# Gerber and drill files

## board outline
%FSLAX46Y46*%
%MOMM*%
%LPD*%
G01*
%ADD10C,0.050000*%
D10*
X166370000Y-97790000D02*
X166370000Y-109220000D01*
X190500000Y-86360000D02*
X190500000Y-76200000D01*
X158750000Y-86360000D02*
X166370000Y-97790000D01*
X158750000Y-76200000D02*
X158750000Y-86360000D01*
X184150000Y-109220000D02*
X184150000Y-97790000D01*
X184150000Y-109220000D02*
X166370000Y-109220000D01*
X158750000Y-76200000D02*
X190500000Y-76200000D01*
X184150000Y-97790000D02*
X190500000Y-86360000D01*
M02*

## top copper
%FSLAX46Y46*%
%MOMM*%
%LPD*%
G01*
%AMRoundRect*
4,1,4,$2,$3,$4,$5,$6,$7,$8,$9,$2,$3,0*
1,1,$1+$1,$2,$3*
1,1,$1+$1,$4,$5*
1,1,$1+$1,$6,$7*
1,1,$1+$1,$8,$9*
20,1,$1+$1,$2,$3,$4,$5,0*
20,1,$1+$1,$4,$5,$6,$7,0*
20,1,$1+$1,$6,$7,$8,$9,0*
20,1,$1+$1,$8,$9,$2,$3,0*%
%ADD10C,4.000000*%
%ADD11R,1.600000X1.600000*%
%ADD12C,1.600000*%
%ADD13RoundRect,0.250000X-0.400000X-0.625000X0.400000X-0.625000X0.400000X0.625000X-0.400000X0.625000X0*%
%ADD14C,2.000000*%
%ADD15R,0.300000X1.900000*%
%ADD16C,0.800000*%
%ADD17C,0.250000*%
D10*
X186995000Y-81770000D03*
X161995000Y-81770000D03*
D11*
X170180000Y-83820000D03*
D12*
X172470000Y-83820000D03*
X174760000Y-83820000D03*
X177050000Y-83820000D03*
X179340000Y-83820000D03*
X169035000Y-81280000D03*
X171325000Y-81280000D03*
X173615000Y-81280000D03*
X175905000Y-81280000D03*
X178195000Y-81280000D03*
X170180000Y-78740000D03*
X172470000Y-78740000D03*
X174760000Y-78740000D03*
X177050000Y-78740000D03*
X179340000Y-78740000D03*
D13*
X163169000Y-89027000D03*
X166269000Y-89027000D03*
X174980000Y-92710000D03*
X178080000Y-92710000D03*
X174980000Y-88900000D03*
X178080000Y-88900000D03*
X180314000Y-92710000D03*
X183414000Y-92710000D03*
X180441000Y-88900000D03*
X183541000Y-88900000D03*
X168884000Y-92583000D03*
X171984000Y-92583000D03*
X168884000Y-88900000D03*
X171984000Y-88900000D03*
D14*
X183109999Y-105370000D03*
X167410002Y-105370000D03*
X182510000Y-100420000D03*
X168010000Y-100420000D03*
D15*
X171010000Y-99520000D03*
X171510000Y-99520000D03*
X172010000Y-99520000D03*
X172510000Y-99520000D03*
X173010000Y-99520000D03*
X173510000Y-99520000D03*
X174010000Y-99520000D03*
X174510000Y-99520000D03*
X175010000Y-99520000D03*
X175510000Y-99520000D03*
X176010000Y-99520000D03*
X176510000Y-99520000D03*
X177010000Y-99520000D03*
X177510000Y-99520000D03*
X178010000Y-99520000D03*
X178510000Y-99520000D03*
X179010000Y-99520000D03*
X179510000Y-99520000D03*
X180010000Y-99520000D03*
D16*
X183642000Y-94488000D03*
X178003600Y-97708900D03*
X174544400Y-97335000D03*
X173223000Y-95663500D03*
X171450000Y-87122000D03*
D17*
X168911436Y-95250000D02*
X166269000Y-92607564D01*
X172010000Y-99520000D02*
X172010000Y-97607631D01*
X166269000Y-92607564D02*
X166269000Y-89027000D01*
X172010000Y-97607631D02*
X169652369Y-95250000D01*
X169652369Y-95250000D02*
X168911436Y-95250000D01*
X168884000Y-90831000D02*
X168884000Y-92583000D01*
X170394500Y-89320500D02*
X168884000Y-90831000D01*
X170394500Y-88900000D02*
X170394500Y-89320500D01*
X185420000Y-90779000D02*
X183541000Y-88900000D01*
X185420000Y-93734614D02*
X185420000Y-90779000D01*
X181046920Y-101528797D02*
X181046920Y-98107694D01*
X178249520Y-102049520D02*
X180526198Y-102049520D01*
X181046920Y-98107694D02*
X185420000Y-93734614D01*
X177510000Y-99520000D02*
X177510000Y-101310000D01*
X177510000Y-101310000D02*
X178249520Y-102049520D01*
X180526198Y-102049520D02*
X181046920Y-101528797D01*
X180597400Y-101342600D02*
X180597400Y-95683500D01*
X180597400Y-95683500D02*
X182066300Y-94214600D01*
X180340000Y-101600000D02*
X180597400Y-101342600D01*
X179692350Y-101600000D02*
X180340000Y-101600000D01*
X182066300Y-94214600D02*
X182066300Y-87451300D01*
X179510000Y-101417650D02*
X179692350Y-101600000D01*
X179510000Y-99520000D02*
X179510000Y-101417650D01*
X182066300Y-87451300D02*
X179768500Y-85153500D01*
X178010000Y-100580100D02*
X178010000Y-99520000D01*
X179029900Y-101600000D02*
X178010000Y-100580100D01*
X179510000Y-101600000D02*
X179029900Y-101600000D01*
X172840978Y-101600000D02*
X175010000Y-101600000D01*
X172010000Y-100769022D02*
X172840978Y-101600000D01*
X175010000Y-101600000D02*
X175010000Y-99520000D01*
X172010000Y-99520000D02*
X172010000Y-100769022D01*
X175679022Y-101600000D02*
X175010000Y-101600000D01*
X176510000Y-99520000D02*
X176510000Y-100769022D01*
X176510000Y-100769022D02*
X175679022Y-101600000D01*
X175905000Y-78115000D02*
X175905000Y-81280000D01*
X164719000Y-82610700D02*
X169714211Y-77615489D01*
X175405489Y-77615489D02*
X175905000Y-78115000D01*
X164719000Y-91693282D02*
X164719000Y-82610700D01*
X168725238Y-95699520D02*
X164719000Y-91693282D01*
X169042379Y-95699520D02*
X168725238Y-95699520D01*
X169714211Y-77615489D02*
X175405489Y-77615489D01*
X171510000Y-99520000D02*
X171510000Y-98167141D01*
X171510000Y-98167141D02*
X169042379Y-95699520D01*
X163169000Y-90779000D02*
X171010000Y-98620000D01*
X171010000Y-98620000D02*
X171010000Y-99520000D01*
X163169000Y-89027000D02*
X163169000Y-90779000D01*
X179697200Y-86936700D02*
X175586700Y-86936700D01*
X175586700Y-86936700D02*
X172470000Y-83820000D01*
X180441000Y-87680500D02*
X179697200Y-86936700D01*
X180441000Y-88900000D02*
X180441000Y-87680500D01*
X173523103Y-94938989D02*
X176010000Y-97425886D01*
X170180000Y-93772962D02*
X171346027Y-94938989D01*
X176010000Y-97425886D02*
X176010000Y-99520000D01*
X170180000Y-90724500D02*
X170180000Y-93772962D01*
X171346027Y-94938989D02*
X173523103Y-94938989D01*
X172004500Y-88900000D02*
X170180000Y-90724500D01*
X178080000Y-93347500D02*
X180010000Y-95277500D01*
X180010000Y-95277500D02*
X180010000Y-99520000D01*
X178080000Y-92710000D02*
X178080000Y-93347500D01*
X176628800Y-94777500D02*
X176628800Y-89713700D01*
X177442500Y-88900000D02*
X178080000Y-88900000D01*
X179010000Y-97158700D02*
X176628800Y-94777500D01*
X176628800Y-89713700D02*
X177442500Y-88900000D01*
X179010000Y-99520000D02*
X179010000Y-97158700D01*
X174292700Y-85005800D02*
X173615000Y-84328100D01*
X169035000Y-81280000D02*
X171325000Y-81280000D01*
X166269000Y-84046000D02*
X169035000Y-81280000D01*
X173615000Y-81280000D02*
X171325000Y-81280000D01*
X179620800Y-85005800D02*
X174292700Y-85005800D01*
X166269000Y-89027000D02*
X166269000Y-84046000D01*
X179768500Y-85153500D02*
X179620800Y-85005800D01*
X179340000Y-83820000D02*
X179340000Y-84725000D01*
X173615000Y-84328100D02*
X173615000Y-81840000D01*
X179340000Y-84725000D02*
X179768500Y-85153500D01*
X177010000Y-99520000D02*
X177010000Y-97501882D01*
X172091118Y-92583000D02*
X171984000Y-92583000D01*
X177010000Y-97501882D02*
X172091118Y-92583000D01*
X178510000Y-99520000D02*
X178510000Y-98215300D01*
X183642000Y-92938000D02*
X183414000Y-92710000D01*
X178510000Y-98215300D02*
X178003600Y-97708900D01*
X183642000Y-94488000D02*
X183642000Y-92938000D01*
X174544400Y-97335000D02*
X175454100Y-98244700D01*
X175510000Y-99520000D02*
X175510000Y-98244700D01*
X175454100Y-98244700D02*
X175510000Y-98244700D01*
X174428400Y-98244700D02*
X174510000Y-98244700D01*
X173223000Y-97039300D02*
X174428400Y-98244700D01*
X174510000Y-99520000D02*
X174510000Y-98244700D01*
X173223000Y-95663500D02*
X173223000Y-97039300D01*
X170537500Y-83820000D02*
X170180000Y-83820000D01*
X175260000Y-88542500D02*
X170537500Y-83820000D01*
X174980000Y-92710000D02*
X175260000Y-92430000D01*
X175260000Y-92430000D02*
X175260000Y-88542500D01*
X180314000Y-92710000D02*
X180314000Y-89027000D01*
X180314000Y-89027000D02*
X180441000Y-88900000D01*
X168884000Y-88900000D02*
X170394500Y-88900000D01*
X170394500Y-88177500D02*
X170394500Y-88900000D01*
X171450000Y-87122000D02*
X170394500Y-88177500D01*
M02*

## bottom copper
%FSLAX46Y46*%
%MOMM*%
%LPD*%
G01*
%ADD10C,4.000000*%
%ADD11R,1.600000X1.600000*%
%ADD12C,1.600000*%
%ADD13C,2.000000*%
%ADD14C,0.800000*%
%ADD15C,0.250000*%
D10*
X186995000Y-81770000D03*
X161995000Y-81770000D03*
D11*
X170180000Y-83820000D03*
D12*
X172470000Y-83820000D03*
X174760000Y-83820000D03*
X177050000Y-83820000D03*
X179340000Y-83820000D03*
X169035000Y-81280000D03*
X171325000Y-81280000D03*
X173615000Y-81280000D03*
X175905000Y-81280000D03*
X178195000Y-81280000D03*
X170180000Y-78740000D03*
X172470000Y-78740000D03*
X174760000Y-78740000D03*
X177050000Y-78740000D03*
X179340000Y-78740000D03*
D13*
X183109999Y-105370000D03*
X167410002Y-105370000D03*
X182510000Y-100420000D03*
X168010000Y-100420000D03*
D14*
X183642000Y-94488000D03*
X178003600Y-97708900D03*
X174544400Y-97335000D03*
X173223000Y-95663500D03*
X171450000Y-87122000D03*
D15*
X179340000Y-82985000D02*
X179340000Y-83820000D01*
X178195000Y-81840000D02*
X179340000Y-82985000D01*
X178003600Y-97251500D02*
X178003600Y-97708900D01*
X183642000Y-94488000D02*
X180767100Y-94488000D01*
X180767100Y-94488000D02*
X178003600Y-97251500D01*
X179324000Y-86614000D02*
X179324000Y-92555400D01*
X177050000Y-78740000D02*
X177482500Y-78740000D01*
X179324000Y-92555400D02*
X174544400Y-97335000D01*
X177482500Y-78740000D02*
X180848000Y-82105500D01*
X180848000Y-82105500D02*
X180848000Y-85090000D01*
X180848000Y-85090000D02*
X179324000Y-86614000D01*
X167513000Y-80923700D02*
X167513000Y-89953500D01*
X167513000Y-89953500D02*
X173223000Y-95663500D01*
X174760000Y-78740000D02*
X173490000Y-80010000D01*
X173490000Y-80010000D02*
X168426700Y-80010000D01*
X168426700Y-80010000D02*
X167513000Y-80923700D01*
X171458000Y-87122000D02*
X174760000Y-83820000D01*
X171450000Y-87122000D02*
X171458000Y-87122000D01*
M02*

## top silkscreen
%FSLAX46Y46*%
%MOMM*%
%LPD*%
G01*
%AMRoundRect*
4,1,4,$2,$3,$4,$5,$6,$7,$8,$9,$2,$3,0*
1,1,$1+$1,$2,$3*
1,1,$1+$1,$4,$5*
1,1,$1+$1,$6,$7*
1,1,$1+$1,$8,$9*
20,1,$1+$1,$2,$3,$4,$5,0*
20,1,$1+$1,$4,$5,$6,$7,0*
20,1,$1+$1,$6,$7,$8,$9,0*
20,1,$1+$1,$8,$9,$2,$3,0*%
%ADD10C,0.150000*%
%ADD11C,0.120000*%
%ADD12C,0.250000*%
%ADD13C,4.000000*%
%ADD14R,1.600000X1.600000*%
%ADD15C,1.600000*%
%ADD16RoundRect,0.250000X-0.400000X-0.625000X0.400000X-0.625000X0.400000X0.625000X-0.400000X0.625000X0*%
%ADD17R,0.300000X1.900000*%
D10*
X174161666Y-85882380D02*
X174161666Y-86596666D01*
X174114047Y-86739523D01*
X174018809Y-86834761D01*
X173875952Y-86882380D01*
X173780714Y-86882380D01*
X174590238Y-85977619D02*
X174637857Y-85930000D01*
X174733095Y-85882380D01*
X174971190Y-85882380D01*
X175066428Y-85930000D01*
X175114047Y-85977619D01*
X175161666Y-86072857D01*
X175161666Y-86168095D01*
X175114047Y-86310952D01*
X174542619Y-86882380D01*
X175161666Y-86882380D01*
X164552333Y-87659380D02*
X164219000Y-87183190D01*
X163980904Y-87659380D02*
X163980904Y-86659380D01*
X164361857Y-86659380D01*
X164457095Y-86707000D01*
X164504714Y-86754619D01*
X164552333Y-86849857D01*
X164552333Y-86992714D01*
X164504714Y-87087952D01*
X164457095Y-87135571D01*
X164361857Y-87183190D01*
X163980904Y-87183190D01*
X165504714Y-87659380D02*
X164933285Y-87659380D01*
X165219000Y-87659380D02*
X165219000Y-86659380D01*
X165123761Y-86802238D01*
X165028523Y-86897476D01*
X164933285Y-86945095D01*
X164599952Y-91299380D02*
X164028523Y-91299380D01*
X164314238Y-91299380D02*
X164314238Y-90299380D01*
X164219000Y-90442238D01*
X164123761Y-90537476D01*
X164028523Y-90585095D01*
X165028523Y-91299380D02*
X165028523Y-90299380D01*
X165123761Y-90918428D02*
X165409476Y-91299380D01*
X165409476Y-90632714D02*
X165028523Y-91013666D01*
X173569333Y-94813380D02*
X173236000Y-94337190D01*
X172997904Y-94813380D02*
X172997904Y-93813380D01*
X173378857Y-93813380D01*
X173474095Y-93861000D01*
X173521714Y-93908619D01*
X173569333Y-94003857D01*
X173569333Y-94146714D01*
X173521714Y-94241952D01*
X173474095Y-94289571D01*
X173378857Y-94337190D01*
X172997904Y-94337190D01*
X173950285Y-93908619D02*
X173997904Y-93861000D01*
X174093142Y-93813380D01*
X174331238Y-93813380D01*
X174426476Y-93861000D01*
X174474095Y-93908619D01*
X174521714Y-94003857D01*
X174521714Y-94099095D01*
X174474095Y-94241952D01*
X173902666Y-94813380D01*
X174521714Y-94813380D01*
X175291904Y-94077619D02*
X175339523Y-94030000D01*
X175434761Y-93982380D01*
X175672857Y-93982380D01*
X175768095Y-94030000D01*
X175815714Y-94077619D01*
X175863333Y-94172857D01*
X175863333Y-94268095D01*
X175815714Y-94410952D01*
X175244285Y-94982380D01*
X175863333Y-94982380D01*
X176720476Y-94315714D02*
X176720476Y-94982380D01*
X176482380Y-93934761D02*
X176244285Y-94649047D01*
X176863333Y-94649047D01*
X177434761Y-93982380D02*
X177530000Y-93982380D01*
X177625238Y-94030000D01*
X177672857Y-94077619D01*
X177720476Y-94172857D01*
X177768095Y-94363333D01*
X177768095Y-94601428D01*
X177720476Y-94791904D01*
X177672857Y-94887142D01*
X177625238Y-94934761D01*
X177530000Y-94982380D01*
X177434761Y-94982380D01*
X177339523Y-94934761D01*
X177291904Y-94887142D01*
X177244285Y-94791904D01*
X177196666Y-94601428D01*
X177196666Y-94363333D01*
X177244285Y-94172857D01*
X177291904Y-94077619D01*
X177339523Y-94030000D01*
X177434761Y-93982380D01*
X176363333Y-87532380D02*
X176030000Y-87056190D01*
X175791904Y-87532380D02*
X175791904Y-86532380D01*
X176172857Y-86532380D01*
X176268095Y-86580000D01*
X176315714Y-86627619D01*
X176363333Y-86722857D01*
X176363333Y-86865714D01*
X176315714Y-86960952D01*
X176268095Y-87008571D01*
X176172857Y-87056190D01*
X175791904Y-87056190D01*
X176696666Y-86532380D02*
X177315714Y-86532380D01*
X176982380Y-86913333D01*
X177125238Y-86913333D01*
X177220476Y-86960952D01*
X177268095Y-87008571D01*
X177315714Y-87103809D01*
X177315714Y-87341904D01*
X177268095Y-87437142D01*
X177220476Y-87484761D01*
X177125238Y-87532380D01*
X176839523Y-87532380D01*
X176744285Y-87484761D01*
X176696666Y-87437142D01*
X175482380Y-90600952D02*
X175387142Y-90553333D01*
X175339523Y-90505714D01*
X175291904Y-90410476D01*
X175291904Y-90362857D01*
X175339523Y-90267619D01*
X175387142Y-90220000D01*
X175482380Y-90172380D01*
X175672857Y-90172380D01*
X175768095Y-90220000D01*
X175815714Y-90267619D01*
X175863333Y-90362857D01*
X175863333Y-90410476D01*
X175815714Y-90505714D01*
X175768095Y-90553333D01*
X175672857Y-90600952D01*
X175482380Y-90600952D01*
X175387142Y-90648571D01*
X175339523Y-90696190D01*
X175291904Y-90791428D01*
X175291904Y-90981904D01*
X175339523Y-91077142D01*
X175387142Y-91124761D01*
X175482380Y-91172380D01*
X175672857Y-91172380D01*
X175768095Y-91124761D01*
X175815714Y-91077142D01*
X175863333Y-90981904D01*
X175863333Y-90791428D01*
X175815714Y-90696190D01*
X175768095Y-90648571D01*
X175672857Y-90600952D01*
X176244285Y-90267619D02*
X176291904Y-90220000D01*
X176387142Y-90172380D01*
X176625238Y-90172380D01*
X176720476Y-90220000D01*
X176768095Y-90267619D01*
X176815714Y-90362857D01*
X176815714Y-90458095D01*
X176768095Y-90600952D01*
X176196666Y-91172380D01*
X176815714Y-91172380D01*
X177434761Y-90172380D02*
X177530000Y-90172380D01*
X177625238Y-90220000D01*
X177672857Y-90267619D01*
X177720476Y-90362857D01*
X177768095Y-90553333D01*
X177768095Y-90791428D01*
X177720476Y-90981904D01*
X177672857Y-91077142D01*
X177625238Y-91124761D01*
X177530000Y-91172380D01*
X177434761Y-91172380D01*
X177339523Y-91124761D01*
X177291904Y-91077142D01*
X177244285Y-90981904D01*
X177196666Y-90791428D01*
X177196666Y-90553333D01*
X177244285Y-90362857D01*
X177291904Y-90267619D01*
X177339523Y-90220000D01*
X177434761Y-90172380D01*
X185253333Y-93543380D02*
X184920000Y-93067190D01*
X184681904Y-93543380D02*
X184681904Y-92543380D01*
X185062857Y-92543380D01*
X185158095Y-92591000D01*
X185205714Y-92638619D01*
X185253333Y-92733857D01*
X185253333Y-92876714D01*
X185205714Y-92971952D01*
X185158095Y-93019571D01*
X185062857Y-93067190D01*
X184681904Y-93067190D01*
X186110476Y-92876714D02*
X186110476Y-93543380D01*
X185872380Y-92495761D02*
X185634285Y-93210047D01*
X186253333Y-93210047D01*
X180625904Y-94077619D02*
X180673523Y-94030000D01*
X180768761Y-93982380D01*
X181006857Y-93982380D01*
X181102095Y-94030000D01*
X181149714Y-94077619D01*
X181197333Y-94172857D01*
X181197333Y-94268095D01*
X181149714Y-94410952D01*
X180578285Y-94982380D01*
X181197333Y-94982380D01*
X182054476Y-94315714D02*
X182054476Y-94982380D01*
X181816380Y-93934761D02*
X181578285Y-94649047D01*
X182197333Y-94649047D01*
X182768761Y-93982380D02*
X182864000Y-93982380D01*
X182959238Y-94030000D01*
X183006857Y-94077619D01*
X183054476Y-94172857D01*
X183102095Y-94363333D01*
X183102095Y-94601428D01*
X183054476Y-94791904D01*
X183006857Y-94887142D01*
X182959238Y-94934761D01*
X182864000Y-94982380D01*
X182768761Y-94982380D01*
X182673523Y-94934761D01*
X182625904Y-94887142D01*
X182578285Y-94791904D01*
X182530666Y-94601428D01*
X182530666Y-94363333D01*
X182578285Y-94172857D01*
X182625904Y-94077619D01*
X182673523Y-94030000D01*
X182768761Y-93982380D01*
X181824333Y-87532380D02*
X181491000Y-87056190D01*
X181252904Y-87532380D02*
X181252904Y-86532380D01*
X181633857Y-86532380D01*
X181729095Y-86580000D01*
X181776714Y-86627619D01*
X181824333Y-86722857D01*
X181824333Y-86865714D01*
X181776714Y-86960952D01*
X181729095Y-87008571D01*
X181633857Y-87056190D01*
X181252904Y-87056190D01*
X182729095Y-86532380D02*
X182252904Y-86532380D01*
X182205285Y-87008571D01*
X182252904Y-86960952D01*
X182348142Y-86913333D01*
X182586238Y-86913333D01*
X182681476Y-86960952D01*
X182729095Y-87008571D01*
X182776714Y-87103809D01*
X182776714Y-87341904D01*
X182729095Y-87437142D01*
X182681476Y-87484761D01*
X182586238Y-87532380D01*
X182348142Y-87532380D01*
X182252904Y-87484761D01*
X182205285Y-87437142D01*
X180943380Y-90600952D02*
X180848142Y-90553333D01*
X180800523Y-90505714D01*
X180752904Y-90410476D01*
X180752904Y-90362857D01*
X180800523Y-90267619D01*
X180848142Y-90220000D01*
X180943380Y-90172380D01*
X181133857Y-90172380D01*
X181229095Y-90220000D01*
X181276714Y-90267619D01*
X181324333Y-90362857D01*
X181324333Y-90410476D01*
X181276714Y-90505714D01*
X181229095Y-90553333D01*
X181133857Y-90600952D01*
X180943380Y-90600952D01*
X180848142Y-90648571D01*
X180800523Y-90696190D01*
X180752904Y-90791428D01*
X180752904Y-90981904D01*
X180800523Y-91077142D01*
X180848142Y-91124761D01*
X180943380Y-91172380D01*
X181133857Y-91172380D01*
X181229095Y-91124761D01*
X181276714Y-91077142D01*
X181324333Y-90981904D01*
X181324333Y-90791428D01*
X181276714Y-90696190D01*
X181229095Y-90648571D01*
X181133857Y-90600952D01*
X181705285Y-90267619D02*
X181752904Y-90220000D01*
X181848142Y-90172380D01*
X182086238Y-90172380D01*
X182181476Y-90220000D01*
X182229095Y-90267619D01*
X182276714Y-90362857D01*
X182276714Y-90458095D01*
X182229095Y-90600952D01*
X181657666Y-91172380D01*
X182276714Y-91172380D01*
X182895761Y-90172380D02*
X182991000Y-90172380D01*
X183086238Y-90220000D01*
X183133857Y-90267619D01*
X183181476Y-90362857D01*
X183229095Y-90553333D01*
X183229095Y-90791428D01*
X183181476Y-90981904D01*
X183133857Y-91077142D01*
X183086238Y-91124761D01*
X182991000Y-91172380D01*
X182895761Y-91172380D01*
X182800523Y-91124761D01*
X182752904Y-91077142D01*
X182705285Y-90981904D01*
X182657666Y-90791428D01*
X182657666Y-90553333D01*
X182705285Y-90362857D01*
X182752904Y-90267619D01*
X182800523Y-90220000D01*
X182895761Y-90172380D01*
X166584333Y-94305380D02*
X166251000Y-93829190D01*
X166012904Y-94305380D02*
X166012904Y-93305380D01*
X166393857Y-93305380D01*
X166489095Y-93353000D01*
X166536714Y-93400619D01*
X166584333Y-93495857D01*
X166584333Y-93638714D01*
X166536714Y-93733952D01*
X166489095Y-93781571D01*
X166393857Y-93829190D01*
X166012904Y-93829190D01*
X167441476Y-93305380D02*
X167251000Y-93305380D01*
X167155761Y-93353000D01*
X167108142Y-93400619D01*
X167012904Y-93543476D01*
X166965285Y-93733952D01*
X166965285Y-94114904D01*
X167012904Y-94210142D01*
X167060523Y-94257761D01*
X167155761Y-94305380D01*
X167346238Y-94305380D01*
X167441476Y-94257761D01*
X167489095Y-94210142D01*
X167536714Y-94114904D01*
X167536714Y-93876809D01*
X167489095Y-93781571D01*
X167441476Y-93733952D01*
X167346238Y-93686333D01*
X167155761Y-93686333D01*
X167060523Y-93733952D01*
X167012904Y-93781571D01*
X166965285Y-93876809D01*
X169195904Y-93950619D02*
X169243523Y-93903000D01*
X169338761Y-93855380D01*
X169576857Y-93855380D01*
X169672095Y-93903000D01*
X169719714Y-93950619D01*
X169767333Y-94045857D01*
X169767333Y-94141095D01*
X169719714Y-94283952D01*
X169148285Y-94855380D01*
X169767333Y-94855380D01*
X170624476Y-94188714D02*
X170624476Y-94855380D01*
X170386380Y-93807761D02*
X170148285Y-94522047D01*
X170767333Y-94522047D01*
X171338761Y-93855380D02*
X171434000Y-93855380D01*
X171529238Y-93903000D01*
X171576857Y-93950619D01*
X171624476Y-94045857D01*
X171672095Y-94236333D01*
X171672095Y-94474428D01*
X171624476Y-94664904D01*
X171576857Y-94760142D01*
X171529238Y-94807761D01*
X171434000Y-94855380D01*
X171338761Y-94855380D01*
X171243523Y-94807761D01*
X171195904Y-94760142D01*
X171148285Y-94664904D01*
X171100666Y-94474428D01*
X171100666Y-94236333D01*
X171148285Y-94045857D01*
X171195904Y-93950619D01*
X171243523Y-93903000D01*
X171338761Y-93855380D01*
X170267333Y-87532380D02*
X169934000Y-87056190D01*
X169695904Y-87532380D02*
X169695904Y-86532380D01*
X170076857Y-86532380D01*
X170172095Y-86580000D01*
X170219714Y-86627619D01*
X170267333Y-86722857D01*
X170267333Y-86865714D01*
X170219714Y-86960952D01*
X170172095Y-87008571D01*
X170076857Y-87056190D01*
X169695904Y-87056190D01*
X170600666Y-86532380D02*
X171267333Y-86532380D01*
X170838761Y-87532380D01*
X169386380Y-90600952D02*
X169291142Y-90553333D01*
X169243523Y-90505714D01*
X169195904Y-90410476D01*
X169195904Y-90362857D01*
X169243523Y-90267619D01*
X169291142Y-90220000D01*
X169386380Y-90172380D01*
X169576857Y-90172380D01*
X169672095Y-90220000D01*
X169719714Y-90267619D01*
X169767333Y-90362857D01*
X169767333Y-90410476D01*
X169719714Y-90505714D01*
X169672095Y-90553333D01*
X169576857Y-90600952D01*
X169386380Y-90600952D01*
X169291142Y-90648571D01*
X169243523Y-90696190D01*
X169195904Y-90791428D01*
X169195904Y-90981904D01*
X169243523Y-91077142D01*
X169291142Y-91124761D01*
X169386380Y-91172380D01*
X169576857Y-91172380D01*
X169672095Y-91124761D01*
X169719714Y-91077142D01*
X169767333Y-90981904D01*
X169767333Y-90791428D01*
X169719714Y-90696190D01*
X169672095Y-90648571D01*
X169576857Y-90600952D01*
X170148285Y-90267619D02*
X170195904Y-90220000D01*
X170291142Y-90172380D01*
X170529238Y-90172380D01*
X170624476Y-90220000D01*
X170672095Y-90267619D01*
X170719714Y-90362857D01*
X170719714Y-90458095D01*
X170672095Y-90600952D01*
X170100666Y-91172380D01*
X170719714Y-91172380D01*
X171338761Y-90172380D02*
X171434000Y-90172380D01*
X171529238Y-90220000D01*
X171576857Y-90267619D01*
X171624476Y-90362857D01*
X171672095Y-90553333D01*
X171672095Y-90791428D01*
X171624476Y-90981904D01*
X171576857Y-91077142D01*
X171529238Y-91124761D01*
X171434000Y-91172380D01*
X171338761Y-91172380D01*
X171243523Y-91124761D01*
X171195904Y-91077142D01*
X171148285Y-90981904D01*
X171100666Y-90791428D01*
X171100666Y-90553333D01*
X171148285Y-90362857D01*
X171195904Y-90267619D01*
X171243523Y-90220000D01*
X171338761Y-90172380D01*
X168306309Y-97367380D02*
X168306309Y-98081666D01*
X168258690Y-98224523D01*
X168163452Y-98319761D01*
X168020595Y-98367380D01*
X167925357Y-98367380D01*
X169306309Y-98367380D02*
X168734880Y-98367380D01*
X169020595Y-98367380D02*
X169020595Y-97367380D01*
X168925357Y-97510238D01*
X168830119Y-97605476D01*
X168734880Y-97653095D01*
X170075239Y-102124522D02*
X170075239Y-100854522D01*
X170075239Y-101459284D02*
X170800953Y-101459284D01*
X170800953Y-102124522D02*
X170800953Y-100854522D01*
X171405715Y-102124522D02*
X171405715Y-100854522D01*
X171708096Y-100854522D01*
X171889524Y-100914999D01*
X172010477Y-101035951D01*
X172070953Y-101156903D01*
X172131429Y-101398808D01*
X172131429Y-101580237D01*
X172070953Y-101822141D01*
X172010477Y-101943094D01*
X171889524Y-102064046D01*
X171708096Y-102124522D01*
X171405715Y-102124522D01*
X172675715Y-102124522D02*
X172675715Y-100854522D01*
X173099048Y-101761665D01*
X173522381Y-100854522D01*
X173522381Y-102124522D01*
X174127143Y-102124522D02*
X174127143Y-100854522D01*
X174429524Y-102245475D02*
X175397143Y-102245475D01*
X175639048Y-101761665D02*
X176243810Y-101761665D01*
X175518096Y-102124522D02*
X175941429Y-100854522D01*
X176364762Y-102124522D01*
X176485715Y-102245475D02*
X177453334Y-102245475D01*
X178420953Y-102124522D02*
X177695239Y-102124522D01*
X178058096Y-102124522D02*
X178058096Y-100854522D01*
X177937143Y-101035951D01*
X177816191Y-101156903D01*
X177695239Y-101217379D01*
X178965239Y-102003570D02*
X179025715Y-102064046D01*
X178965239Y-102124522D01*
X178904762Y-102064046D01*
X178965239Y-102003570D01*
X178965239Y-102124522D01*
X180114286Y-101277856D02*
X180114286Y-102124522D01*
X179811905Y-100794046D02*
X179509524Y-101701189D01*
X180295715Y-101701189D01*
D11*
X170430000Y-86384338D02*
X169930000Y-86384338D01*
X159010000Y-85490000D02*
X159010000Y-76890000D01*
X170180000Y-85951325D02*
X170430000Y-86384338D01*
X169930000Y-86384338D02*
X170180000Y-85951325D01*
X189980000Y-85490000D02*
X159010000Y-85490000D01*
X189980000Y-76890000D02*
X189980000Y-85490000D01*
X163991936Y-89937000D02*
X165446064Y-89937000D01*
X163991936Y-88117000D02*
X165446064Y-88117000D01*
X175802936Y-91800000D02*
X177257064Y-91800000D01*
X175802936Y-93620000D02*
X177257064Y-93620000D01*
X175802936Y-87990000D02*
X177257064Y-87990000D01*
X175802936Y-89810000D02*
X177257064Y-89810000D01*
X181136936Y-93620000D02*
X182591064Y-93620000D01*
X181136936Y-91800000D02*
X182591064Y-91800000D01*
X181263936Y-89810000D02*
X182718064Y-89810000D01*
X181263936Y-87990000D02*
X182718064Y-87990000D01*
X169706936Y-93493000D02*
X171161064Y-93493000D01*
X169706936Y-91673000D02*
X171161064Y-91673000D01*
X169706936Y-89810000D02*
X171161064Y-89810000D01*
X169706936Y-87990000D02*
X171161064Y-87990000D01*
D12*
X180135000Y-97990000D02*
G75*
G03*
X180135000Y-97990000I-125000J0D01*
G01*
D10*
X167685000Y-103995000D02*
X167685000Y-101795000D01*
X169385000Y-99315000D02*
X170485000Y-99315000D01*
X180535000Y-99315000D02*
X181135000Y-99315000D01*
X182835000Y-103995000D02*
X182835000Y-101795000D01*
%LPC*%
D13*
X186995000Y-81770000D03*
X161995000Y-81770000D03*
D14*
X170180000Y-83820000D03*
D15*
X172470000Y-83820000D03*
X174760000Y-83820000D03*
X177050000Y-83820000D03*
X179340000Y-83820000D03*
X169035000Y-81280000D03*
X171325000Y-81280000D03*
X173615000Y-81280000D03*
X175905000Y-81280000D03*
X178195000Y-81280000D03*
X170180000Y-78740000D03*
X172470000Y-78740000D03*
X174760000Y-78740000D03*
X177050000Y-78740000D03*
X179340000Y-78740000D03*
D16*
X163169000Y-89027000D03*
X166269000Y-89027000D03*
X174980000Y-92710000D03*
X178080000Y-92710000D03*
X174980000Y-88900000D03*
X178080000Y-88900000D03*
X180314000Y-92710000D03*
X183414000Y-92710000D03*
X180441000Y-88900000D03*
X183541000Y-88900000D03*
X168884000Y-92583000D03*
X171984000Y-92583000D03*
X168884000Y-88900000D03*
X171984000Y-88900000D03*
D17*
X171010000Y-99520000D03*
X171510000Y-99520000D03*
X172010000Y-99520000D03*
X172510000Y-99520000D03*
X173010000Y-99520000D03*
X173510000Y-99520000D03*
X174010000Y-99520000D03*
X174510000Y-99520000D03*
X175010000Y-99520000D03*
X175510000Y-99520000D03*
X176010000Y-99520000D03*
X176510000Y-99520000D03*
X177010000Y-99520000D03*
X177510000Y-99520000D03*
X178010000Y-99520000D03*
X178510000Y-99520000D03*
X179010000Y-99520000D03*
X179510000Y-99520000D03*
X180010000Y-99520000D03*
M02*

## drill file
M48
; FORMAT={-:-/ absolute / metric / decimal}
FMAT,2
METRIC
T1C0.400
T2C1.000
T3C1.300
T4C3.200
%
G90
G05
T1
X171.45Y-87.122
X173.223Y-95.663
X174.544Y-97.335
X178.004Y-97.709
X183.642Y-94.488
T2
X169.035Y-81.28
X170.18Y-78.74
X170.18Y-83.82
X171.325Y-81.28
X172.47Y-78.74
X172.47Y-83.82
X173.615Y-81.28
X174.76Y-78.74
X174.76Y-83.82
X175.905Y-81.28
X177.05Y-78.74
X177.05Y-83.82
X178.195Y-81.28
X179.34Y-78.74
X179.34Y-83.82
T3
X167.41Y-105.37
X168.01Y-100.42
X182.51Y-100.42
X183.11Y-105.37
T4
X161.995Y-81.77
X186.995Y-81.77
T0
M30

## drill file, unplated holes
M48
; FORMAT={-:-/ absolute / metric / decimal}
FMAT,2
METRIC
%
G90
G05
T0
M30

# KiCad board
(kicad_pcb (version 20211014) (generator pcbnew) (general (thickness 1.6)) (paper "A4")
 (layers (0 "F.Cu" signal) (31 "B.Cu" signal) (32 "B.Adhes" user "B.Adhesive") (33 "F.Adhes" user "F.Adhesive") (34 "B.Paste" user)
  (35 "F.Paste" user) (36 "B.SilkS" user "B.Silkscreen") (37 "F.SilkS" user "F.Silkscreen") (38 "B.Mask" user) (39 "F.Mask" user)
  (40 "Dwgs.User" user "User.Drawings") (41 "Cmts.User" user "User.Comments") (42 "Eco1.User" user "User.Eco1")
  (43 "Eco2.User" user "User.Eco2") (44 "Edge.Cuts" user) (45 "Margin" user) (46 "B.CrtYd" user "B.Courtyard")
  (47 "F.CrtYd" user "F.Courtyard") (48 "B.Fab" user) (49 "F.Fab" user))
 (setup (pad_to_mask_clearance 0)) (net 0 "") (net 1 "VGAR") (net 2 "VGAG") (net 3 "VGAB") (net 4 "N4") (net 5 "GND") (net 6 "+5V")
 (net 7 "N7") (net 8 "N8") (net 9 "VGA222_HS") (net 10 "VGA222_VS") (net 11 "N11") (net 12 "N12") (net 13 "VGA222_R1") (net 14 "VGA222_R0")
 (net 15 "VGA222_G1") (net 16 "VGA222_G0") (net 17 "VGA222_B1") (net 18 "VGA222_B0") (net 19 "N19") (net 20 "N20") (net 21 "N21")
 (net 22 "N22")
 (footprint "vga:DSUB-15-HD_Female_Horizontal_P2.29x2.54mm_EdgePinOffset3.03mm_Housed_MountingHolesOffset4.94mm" (layer "F.Cu")
  (at 170.18 83.82 180)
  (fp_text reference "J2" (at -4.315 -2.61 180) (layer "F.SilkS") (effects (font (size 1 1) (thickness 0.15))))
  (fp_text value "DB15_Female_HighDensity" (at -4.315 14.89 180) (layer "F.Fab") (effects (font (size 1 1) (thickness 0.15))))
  (fp_line (start -0.25 -2.564338) (end 0.25 -2.564338) (layer "F.SilkS") (width 0.12))
  (fp_line (start 11.17 -1.67) (end 11.17 6.93) (layer "F.SilkS") (width 0.12))
  (fp_line (start 0 -2.131325) (end -0.25 -2.564338) (layer "F.SilkS") (width 0.12))
  (fp_line (start 0.25 -2.564338) (end 0 -2.131325) (layer "F.SilkS") (width 0.12))
  (fp_line (start -19.8 -1.67) (end 11.17 -1.67) (layer "F.SilkS") (width 0.12))
  (fp_line (start -19.8 6.93) (end -19.8 -1.67) (layer "F.SilkS") (width 0.12))
  (pad "0" thru_hole circle (at -16.815 2.05 180) (size 4 4) (drill 3.2) (layers *.Cu *.Mask))
  (pad "0" thru_hole circle (at 8.185 2.05 180) (size 4 4) (drill 3.2) (layers *.Cu *.Mask))
  (pad "1" thru_hole rect (at 0 0 180) (size 1.6 1.6) (drill 1) (layers *.Cu *.Mask) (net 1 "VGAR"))
  (pad "2" thru_hole circle (at -2.29 0 180) (size 1.6 1.6) (drill 1) (layers *.Cu *.Mask) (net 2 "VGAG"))
  (pad "3" thru_hole circle (at -4.58 0 180) (size 1.6 1.6) (drill 1) (layers *.Cu *.Mask) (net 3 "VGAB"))
  (pad "4" thru_hole circle (at -6.87 0 180) (size 1.6 1.6) (drill 1) (layers *.Cu *.Mask) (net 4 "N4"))
  (pad "5" thru_hole circle (at -9.16 0 180) (size 1.6 1.6) (drill 1) (layers *.Cu *.Mask) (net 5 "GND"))
  (pad "6" thru_hole circle (at 1.145 2.54 180) (size 1.6 1.6) (drill 1) (layers *.Cu *.Mask) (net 5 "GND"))
  (pad "7" thru_hole circle (at -1.145 2.54 180) (size 1.6 1.6) (drill 1) (layers *.Cu *.Mask) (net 5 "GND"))
  (pad "8" thru_hole circle (at -3.435 2.54 180) (size 1.6 1.6) (drill 1) (layers *.Cu *.Mask) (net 5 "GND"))
  (pad "9" thru_hole circle (at -5.725 2.54 180) (size 1.6 1.6) (drill 1) (layers *.Cu *.Mask) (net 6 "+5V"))
  (pad "10" thru_hole circle (at -8.015 2.54 180) (size 1.6 1.6) (drill 1) (layers *.Cu *.Mask) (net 5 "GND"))
  (pad "11" thru_hole circle (at 0 5.08 180) (size 1.6 1.6) (drill 1) (layers *.Cu *.Mask) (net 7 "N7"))
  (pad "12" thru_hole circle (at -2.29 5.08 180) (size 1.6 1.6) (drill 1) (layers *.Cu *.Mask) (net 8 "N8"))
  (pad "13" thru_hole circle (at -4.58 5.08 180) (size 1.6 1.6) (drill 1) (layers *.Cu *.Mask) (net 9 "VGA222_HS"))
  (pad "14" thru_hole circle (at -6.87 5.08 180) (size 1.6 1.6) (drill 1) (layers *.Cu *.Mask) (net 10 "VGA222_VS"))
  (pad "15" thru_hole circle (at -9.16 5.08 180) (size 1.6 1.6) (drill 1) (layers *.Cu *.Mask) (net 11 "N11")))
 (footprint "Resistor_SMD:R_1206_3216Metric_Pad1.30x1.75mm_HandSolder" (layer "F.Cu") (at 164.719 89.027)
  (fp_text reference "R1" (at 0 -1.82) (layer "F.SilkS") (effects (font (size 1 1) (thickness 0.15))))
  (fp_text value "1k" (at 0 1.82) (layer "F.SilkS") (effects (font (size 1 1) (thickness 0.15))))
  (fp_line (start -0.727064 0.91) (end 0.727064 0.91) (layer "F.SilkS") (width 0.12))
  (fp_line (start -0.727064 -0.91) (end 0.727064 -0.91) (layer "F.SilkS") (width 0.12))
  (pad "1" smd roundrect locked (at -1.55 0) (size 1.3 1.75) (layers "F.Cu" "F.Paste" "F.Mask") (roundrect_rratio 0.1923076923)
   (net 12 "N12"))
  (pad "2" smd roundrect locked (at 1.55 0) (size 1.3 1.75) (layers "F.Cu" "F.Paste" "F.Mask") (roundrect_rratio 0.1923076923) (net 5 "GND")))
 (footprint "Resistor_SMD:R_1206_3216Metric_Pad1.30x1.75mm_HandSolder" (layer "F.Cu") (at 176.53 92.71)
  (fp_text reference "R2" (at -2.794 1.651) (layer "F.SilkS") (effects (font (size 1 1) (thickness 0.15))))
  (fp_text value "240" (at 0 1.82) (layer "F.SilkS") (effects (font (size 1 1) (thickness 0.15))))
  (fp_line (start -0.727064 -0.91) (end 0.727064 -0.91) (layer "F.SilkS") (width 0.12))
  (fp_line (start -0.727064 0.91) (end 0.727064 0.91) (layer "F.SilkS") (width 0.12))
  (pad "1" smd roundrect locked (at -1.55 0) (size 1.3 1.75) (layers "F.Cu" "F.Paste" "F.Mask") (roundrect_rratio 0.1923076923)
   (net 1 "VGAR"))
  (pad "2" smd roundrect locked (at 1.55 0) (size 1.3 1.75) (layers "F.Cu" "F.Paste" "F.Mask") (roundrect_rratio 0.1923076923)
   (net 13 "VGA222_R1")))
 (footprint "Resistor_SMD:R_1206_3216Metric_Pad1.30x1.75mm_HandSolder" (layer "F.Cu") (at 176.53 88.9)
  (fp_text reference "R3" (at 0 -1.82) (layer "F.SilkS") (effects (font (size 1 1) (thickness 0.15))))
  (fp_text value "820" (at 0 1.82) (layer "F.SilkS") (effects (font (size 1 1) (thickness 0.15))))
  (fp_line (start -0.727064 -0.91) (end 0.727064 -0.91) (layer "F.SilkS") (width 0.12))
  (fp_line (start -0.727064 0.91) (end 0.727064 0.91) (layer "F.SilkS") (width 0.12))
  (pad "1" smd roundrect locked (at -1.55 0) (size 1.3 1.75) (layers "F.Cu" "F.Paste" "F.Mask") (roundrect_rratio 0.1923076923)
   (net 1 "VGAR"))
  (pad "2" smd roundrect locked (at 1.55 0) (size 1.3 1.75) (layers "F.Cu" "F.Paste" "F.Mask") (roundrect_rratio 0.1923076923)
   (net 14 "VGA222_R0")))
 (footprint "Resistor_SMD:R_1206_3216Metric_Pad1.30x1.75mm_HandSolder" (layer "F.Cu") (at 181.864 92.71)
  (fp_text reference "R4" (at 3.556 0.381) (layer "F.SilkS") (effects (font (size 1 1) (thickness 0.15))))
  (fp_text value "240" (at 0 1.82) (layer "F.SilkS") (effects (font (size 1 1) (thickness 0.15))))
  (fp_line (start -0.727064 0.91) (end 0.727064 0.91) (layer "F.SilkS") (width 0.12))
  (fp_line (start -0.727064 -0.91) (end 0.727064 -0.91) (layer "F.SilkS") (width 0.12))
  (pad "1" smd roundrect locked (at -1.55 0) (size 1.3 1.75) (layers "F.Cu" "F.Paste" "F.Mask") (roundrect_rratio 0.1923076923)
   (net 2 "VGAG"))
  (pad "2" smd roundrect locked (at 1.55 0) (size 1.3 1.75) (layers "F.Cu" "F.Paste" "F.Mask") (roundrect_rratio 0.1923076923)
   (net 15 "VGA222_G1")))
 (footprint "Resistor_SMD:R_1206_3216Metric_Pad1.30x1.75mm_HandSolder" (layer "F.Cu") (at 181.991 88.9)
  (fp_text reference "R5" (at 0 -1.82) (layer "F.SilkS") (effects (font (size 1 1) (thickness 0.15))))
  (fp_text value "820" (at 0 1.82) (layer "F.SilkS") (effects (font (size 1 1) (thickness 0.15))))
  (fp_line (start -0.727064 0.91) (end 0.727064 0.91) (layer "F.SilkS") (width 0.12))
  (fp_line (start -0.727064 -0.91) (end 0.727064 -0.91) (layer "F.SilkS") (width 0.12))
  (pad "1" smd roundrect locked (at -1.55 0) (size 1.3 1.75) (layers "F.Cu" "F.Paste" "F.Mask") (roundrect_rratio 0.1923076923)
   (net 2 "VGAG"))
  (pad "2" smd roundrect locked (at 1.55 0) (size 1.3 1.75) (layers "F.Cu" "F.Paste" "F.Mask") (roundrect_rratio 0.1923076923)
   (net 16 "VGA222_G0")))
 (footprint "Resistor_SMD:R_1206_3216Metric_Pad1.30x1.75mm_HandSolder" (layer "F.Cu") (at 170.434 92.583)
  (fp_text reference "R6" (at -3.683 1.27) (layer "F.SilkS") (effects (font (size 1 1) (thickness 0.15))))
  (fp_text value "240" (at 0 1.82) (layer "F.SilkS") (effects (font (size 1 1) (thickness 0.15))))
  (fp_line (start -0.727064 0.91) (end 0.727064 0.91) (layer "F.SilkS") (width 0.12))
  (fp_line (start -0.727064 -0.91) (end 0.727064 -0.91) (layer "F.SilkS") (width 0.12))
  (pad "1" smd roundrect locked (at -1.55 0) (size 1.3 1.75) (layers "F.Cu" "F.Paste" "F.Mask") (roundrect_rratio 0.1923076923)
   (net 3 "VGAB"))
  (pad "2" smd roundrect locked (at 1.55 0) (size 1.3 1.75) (layers "F.Cu" "F.Paste" "F.Mask") (roundrect_rratio 0.1923076923)
   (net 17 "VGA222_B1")))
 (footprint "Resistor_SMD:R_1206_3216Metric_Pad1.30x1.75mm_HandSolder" (layer "F.Cu") (at 170.434 88.9)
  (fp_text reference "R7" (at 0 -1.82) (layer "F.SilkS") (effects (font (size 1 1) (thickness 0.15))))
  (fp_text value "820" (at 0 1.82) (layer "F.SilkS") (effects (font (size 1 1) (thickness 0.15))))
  (fp_line (start -0.727064 0.91) (end 0.727064 0.91) (layer "F.SilkS") (width 0.12))
  (fp_line (start -0.727064 -0.91) (end 0.727064 -0.91) (layer "F.SilkS") (width 0.12))
  (pad "1" smd roundrect locked (at -1.55 0) (size 1.3 1.75) (layers "F.Cu" "F.Paste" "F.Mask") (roundrect_rratio 0.1923076923)
   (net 3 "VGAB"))
  (pad "2" smd roundrect locked (at 1.55 0) (size 1.3 1.75) (layers "F.Cu" "F.Paste" "F.Mask") (roundrect_rratio 0.1923076923)
   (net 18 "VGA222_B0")))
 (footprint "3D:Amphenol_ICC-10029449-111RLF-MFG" (layer "F.Cu") (at 175.26 104.14)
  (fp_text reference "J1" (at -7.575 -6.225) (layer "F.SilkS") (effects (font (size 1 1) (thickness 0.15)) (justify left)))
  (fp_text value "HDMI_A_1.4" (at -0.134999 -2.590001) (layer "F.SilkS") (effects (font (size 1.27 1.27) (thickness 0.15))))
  (fp_line (start 7.575 -0.145) (end 7.575 -2.345) (layer "F.SilkS") (width 0.15))
  (fp_line (start 5.275 -4.825) (end 5.875 -4.825) (layer "F.SilkS") (width 0.15))
  (fp_line (start -5.875 -4.825) (end -4.775 -4.825) (layer "F.SilkS") (width 0.15))
  (fp_line (start -7.575 -0.145) (end -7.575 -2.345) (layer "F.SilkS") (width 0.15))
  (fp_circle (center 4.75 -6.15) (end 4.875 -6.15) (layer "F.SilkS") (width 0.25) (fill none))
  (pad "1" smd rect locked (at 4.75 -4.62) (size 0.3 1.9) (layers "F.Cu" "F.Paste" "F.Mask") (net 13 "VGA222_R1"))
  (pad "2" smd rect locked (at 4.25 -4.62) (size 0.3 1.9) (layers "F.Cu" "F.Paste" "F.Mask") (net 5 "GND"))
  (pad "3" smd rect locked (at 3.75 -4.62) (size 0.3 1.9) (layers "F.Cu" "F.Paste" "F.Mask") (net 14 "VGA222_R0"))
  (pad "4" smd rect locked (at 3.25 -4.62) (size 0.3 1.9) (layers "F.Cu" "F.Paste" "F.Mask") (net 15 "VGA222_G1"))
  (pad "5" smd rect locked (at 2.75 -4.62) (size 0.3 1.9) (layers "F.Cu" "F.Paste" "F.Mask") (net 5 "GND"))
  (pad "6" smd rect locked (at 2.25 -4.62) (size 0.3 1.9) (layers "F.Cu" "F.Paste" "F.Mask") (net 16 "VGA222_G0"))
  (pad "7" smd rect locked (at 1.75 -4.62) (size 0.3 1.9) (layers "F.Cu" "F.Paste" "F.Mask") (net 17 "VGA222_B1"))
  (pad "8" smd rect locked (at 1.25 -4.62) (size 0.3 1.9) (layers "F.Cu" "F.Paste" "F.Mask") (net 5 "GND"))
  (pad "9" smd rect locked (at 0.75 -4.62) (size 0.3 1.9) (layers "F.Cu" "F.Paste" "F.Mask") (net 18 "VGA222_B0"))
  (pad "10" smd rect locked (at 0.25 -4.62) (size 0.3 1.9) (layers "F.Cu" "F.Paste" "F.Mask") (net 10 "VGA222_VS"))
  (pad "11" smd rect locked (at -0.25 -4.62) (size 0.3 1.9) (layers "F.Cu" "F.Paste" "F.Mask") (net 5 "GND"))
  (pad "12" smd rect locked (at -0.75 -4.62) (size 0.3 1.9) (layers "F.Cu" "F.Paste" "F.Mask") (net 9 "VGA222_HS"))
  (pad "13" smd rect locked (at -1.25 -4.62) (size 0.3 1.9) (layers "F.Cu" "F.Paste" "F.Mask") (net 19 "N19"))
  (pad "14" smd rect locked (at -1.75 -4.62) (size 0.3 1.9) (layers "F.Cu" "F.Paste" "F.Mask") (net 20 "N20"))
  (pad "15" smd rect locked (at -2.25 -4.62) (size 0.3 1.9) (layers "F.Cu" "F.Paste" "F.Mask") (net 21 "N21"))
  (pad "16" smd rect locked (at -2.75 -4.62) (size 0.3 1.9) (layers "F.Cu" "F.Paste" "F.Mask") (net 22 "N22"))
  (pad "17" smd rect locked (at -3.25 -4.62) (size 0.3 1.9) (layers "F.Cu" "F.Paste" "F.Mask") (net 5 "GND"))
  (pad "18" smd rect locked (at -3.75 -4.62) (size 0.3 1.9) (layers "F.Cu" "F.Paste" "F.Mask") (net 6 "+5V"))
  (pad "19" smd rect locked (at -4.25 -4.62) (size 0.3 1.9) (layers "F.Cu" "F.Paste" "F.Mask") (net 12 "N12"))
  (pad "20" thru_hole circle locked (at -7.25 -3.72) (size 2 2) (drill 1.3) (layers *.Cu))
  (pad "21" thru_hole circle locked (at 7.25 -3.72) (size 2 2) (drill 1.3) (layers *.Cu))
  (pad "22" thru_hole circle locked (at -7.849998 1.23) (size 2 2) (drill 1.3) (layers *.Cu))
  (pad "23" thru_hole circle locked (at 7.849999 1.23) (size 2 2) (drill 1.3) (layers *.Cu)))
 (gr_line (start 166.37 97.79) (end 166.37 109.22) (layer "Edge.Cuts") (width 0.05))
 (gr_line (start 190.5 86.36) (end 190.5 76.2) (layer "Edge.Cuts") (width 0.05))
 (gr_line (start 158.75 86.36) (end 166.37 97.79) (layer "Edge.Cuts") (width 0.05))
 (gr_line (start 158.75 76.2) (end 158.75 86.36) (layer "Edge.Cuts") (width 0.05))
 (gr_line (start 184.15 109.22) (end 184.15 97.79) (layer "Edge.Cuts") (width 0.05))
 (gr_line (start 184.15 109.22) (end 166.37 109.22) (layer "Edge.Cuts") (width 0.05))
 (gr_line (start 158.75 76.2) (end 190.5 76.2) (layer "Edge.Cuts") (width 0.05))
 (gr_line (start 184.15 97.79) (end 190.5 86.36) (layer "Edge.Cuts") (width 0.05))
 (segment (start 171.01 98.62) (end 171.01 99.52) (width 0.25) (layer "F.Cu") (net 12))
 (segment (start 163.169 90.779) (end 171.01 98.62) (width 0.25) (layer "F.Cu") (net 12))
 (segment (start 163.169 89.027) (end 163.169 90.779) (width 0.25) (layer "F.Cu") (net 12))
 (segment (start 178.08 93.3475) (end 180.01 95.2775) (width 0.25) (layer "F.Cu") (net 13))
 (segment (start 180.01 95.2775) (end 180.01 99.52) (width 0.25) (layer "F.Cu") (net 13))
 (segment (start 178.08 92.71) (end 178.08 93.3475) (width 0.25) (layer "F.Cu") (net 13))
 (segment (start 176.6288 94.7775) (end 176.6288 89.7137) (width 0.25) (layer "F.Cu") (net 14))
 (segment (start 177.4425 88.9) (end 178.08 88.9) (width 0.25) (layer "F.Cu") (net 14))
 (segment (start 179.01 97.1587) (end 176.6288 94.7775) (width 0.25) (layer "F.Cu") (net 14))
 (segment (start 176.6288 89.7137) (end 177.4425 88.9) (width 0.25) (layer "F.Cu") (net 14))
 (segment (start 179.01 99.52) (end 179.01 97.1587) (width 0.25) (layer "F.Cu") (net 14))
 (segment (start 174.2927 85.0058) (end 173.615 84.3281) (width 0.25) (layer "F.Cu") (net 5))
 (segment (start 166.269 92.607564) (end 166.269 89.027) (width 0.25) (layer "F.Cu") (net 5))
 (segment (start 182.0663 94.2146) (end 182.0663 87.4513) (width 0.25) (layer "F.Cu") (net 5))
 (segment (start 179.0299 101.6) (end 178.01 100.5801) (width 0.25) (layer "F.Cu") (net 5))
 (segment (start 169.035 81.28) (end 171.325 81.28) (width 0.25) (layer "F.Cu") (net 5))
 (segment (start 166.269 84.046) (end 169.035 81.28) (width 0.25) (layer "F.Cu") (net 5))
 (segment (start 175.679022 101.6) (end 175.01 101.6) (width 0.25) (layer "F.Cu") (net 5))
 (segment (start 179.51 101.6) (end 179.0299 101.6) (width 0.25) (layer "F.Cu") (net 5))
 (segment (start 173.615 81.28) (end 171.325 81.28) (width 0.25) (layer "F.Cu") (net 5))
 (segment (start 178.01 100.5801) (end 178.01 99.52) (width 0.25) (layer "F.Cu") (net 5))
 (segment (start 179.6208 85.0058) (end 174.2927 85.0058) (width 0.25) (layer "F.Cu") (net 5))
 (segment (start 166.269 89.027) (end 166.269 84.046) (width 0.25) (layer "F.Cu") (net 5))
 (segment (start 180.34 101.6) (end 180.5974 101.3426) (width 0.25) (layer "F.Cu") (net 5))
 (segment (start 180.5974 95.6835) (end 182.0663 94.2146) (width 0.25) (layer "F.Cu") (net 5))
 (segment (start 175.01 101.6) (end 175.01 99.52) (width 0.25) (layer "F.Cu") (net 5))
 (segment (start 179.7685 85.1535) (end 179.6208 85.0058) (width 0.25) (layer "F.Cu") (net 5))
 (segment (start 172.01 100.769022) (end 172.840978 101.6) (width 0.25) (layer "F.Cu") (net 5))
 (segment (start 179.51 99.52) (end 179.51 101.41765) (width 0.25) (layer "F.Cu") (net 5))
 (segment (start 172.01 99.52) (end 172.01 100.769022) (width 0.25) (layer "F.Cu") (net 5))
 (segment (start 176.51 99.52) (end 176.51 100.769022) (width 0.25) (layer "F.Cu") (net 5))
 (segment (start 172.840978 101.6) (end 175.01 101.6) (width 0.25) (layer "F.Cu") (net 5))
 (segment (start 179.34 83.82) (end 179.34 84.725) (width 0.25) (layer "F.Cu") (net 5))
 (segment (start 172.01 97.607631) (end 169.652369 95.25) (width 0.25) (layer "F.Cu") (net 5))
 (segment (start 168.911436 95.25) (end 166.269 92.607564) (width 0.25) (layer "F.Cu") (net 5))
 (segment (start 172.01 99.52) (end 172.01 97.607631) (width 0.25) (layer "F.Cu") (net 5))
 (segment (start 179.69235 101.6) (end 180.34 101.6) (width 0.25) (layer "F.Cu") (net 5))
 (segment (start 173.615 84.3281) (end 173.615 81.84) (width 0.25) (layer "F.Cu") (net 5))
 (segment (start 179.51 101.41765) (end 179.69235 101.6) (width 0.25) (layer "F.Cu") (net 5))
 (segment (start 169.652369 95.25) (end 168.911436 95.25) (width 0.25) (layer "F.Cu") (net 5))
 (segment (start 179.34 84.725) (end 179.7685 85.1535) (width 0.25) (layer "F.Cu") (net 5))
 (segment (start 176.51 100.769022) (end 175.679022 101.6) (width 0.25) (layer "F.Cu") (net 5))
 (segment (start 182.0663 87.4513) (end 179.7685 85.1535) (width 0.25) (layer "F.Cu") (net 5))
 (segment (start 180.5974 101.3426) (end 180.5974 95.6835) (width 0.25) (layer "F.Cu") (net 5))
 (segment (start 179.34 82.985) (end 179.34 83.82) (width 0.25) (layer "B.Cu") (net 5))
 (segment (start 178.195 81.84) (end 179.34 82.985) (width 0.25) (layer "B.Cu") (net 5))
 (segment (start 177.01 99.52) (end 177.01 97.501882) (width 0.25) (layer "F.Cu") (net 17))
 (segment (start 172.091118 92.583) (end 171.984 92.583) (width 0.25) (layer "F.Cu") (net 17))
 (segment (start 177.01 97.501882) (end 172.091118 92.583) (width 0.25) (layer "F.Cu") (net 17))
 (segment (start 176.01 97.425886) (end 176.01 99.52) (width 0.25) (layer "F.Cu") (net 18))
 (segment (start 173.523103 94.938989) (end 176.01 97.425886) (width 0.25) (layer "F.Cu") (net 18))
 (segment (start 170.18 90.7245) (end 170.18 93.772962) (width 0.25) (layer "F.Cu") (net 18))
 (segment (start 170.18 93.772962) (end 171.346027 94.938989) (width 0.25) (layer "F.Cu") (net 18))
 (segment (start 171.346027 94.938989) (end 173.523103 94.938989) (width 0.25) (layer "F.Cu") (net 18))
 (segment (start 172.0045 88.9) (end 170.18 90.7245) (width 0.25) (layer "F.Cu") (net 18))
 (segment (start 178.51 99.52) (end 178.51 98.2153) (width 0.25) (layer "F.Cu") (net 15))
 (segment (start 183.642 92.938) (end 183.414 92.71) (width 0.25) (layer "F.Cu") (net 15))
 (segment (start 178.51 98.2153) (end 178.0036 97.7089) (width 0.25) (layer "F.Cu") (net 15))
 (segment (start 183.642 94.488) (end 183.642 92.938) (width 0.25) (layer "F.Cu") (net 15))
 (via (at 183.642 94.488) (size 0.8) (drill 0.4) (layers "F.Cu" "B.Cu") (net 15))
 (via (at 178.0036 97.7089) (size 0.8) (drill 0.4) (layers "F.Cu" "B.Cu") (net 15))
 (segment (start 178.0036 97.2515) (end 178.0036 97.7089) (width 0.25) (layer "B.Cu") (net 15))
 (segment (start 183.642 94.488) (end 180.7671 94.488) (width 0.25) (layer "B.Cu") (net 15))
 (segment (start 180.7671 94.488) (end 178.0036 97.2515) (width 0.25) (layer "B.Cu") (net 15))
 (segment (start 177.51 99.52) (end 177.51 101.31) (width 0.25) (layer "F.Cu") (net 16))
 (segment (start 185.42 90.779) (end 183.541 88.9) (width 0.25) (layer "F.Cu") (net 16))
 (segment (start 177.51 101.31) (end 178.24952 102.04952) (width 0.25) (layer "F.Cu") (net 16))
 (segment (start 180.526198 102.04952) (end 181.04692 101.528797) (width 0.25) (layer "F.Cu") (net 16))
 (segment (start 181.04692 98.107694) (end 185.42 93.734614) (width 0.25) (layer "F.Cu") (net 16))
 (segment (start 185.42 93.734614) (end 185.42 90.779) (width 0.25) (layer "F.Cu") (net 16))
 (segment (start 178.24952 102.04952) (end 180.526198 102.04952) (width 0.25) (layer "F.Cu") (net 16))
 (segment (start 181.04692 101.528797) (end 181.04692 98.107694) (width 0.25) (layer "F.Cu") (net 16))
 (segment (start 174.5444 97.335) (end 175.4541 98.2447) (width 0.25) (layer "F.Cu") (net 10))
 (segment (start 175.51 99.52) (end 175.51 98.2447) (width 0.25) (layer "F.Cu") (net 10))
 (segment (start 175.4541 98.2447) (end 175.51 98.2447) (width 0.25) (layer "F.Cu") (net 10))
 (via (at 174.5444 97.335) (size 0.8) (drill 0.4) (layers "F.Cu" "B.Cu") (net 10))
 (segment (start 179.324 86.614) (end 179.324 92.5554) (width 0.25) (layer "B.Cu") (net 10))
 (segment (start 177.05 78.74) (end 177.4825 78.74) (width 0.25) (layer "B.Cu") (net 10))
 (segment (start 179.324 92.5554) (end 174.5444 97.335) (width 0.25) (layer "B.Cu") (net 10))
 (segment (start 177.4825 78.74) (end 180.848 82.1055) (width 0.25) (layer "B.Cu") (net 10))
 (segment (start 180.848 82.1055) (end 180.848 85.09) (width 0.25) (layer "B.Cu") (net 10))
 (segment (start 180.848 85.09) (end 179.324 86.614) (width 0.25) (layer "B.Cu") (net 10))
 (segment (start 174.4284 98.2447) (end 174.51 98.2447) (width 0.25) (layer "F.Cu") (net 9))
 (segment (start 173.223 97.0393) (end 174.4284 98.2447) (width 0.25) (layer "F.Cu") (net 9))
 (segment (start 174.51 99.52) (end 174.51 98.2447) (width 0.25) (layer "F.Cu") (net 9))
 (segment (start 173.223 95.6635) (end 173.223 97.0393) (width 0.25) (layer "F.Cu") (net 9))
 (via (at 173.223 95.6635) (size 0.8) (drill 0.4) (layers "F.Cu" "B.Cu") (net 9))
 (segment (start 167.513 80.9237) (end 167.513 89.9535) (width 0.25) (layer "B.Cu") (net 9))
 (segment (start 167.513 89.9535) (end 173.223 95.6635) (width 0.25) (layer "B.Cu") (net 9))
 (segment (start 174.76 78.74) (end 173.49 80.01) (width 0.25) (layer "B.Cu") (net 9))
 (segment (start 173.49 80.01) (end 168.4267 80.01) (width 0.25) (layer "B.Cu") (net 9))
 (segment (start 168.4267 80.01) (end 167.513 80.9237) (width 0.25) (layer "B.Cu") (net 9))
 (segment (start 171.51 99.52) (end 171.51 98.167141) (width 0.25) (layer "F.Cu") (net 6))
 (segment (start 171.51 98.167141) (end 169.042379 95.69952) (width 0.25) (layer "F.Cu") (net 6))
 (segment (start 168.725238 95.69952) (end 164.719 91.693282) (width 0.25) (layer "F.Cu") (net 6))
 (segment (start 164.719 82.6107) (end 169.714211 77.615489) (width 0.25) (layer "F.Cu") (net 6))
 (segment (start 164.719 91.693282) (end 164.719 82.6107) (width 0.25) (layer "F.Cu") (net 6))
 (segment (start 175.405489 77.615489) (end 175.905 78.115) (width 0.25) (layer "F.Cu") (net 6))
 (segment (start 175.905 78.115) (end 175.905 81.28) (width 0.25) (layer "F.Cu") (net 6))
 (segment (start 169.714211 77.615489) (end 175.405489 77.615489) (width 0.25) (layer "F.Cu") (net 6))
 (segment (start 169.042379 95.69952) (end 168.725238 95.69952) (width 0.25) (layer "F.Cu") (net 6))
 (segment (start 170.5375 83.82) (end 170.18 83.82) (width 0.25) (layer "F.Cu") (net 1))
 (segment (start 175.26 88.5425) (end 170.5375 83.82) (width 0.25) (layer "F.Cu") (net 1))
 (segment (start 174.98 92.71) (end 175.26 92.43) (width 0.25) (layer "F.Cu") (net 1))
 (segment (start 175.26 92.43) (end 175.26 88.5425) (width 0.25) (layer "F.Cu") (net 1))
 (segment (start 180.314 92.71) (end 180.314 89.027) (width 0.25) (layer "F.Cu") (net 2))
 (segment (start 179.6972 86.9367) (end 175.5867 86.9367) (width 0.25) (layer "F.Cu") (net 2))
 (segment (start 180.441 88.9) (end 180.441 87.6805) (width 0.25) (layer "F.Cu") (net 2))
 (segment (start 180.441 87.6805) (end 179.6972 86.9367) (width 0.25) (layer "F.Cu") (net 2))
 (segment (start 180.314 89.027) (end 180.441 88.9) (width 0.25) (layer "F.Cu") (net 2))
 (segment (start 175.5867 86.9367) (end 172.47 83.82) (width 0.25) (layer "F.Cu") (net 2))
 (segment (start 170.3945 89.3205) (end 168.884 90.831) (width 0.25) (layer "F.Cu") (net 3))
 (segment (start 168.884 88.9) (end 170.3945 88.9) (width 0.25) (layer "F.Cu") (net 3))
 (segment (start 170.3945 88.9) (end 170.3945 89.3205) (width 0.25) (layer "F.Cu") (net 3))
 (segment (start 168.884 90.831) (end 168.884 92.583) (width 0.25) (layer "F.Cu") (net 3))
 (segment (start 170.3945 88.1775) (end 170.3945 88.9) (width 0.25) (layer "F.Cu") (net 3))
 (segment (start 171.45 87.122) (end 170.3945 88.1775) (width 0.25) (layer "F.Cu") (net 3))
 (via (at 171.45 87.122) (size 0.8) (drill 0.4) (layers "F.Cu" "B.Cu") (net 3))
 (segment (start 171.458 87.122) (end 174.76 83.82) (width 0.25) (layer "B.Cu") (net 3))
 (segment (start 171.45 87.122) (end 171.458 87.122) (width 0.25) (layer "B.Cu") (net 3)))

